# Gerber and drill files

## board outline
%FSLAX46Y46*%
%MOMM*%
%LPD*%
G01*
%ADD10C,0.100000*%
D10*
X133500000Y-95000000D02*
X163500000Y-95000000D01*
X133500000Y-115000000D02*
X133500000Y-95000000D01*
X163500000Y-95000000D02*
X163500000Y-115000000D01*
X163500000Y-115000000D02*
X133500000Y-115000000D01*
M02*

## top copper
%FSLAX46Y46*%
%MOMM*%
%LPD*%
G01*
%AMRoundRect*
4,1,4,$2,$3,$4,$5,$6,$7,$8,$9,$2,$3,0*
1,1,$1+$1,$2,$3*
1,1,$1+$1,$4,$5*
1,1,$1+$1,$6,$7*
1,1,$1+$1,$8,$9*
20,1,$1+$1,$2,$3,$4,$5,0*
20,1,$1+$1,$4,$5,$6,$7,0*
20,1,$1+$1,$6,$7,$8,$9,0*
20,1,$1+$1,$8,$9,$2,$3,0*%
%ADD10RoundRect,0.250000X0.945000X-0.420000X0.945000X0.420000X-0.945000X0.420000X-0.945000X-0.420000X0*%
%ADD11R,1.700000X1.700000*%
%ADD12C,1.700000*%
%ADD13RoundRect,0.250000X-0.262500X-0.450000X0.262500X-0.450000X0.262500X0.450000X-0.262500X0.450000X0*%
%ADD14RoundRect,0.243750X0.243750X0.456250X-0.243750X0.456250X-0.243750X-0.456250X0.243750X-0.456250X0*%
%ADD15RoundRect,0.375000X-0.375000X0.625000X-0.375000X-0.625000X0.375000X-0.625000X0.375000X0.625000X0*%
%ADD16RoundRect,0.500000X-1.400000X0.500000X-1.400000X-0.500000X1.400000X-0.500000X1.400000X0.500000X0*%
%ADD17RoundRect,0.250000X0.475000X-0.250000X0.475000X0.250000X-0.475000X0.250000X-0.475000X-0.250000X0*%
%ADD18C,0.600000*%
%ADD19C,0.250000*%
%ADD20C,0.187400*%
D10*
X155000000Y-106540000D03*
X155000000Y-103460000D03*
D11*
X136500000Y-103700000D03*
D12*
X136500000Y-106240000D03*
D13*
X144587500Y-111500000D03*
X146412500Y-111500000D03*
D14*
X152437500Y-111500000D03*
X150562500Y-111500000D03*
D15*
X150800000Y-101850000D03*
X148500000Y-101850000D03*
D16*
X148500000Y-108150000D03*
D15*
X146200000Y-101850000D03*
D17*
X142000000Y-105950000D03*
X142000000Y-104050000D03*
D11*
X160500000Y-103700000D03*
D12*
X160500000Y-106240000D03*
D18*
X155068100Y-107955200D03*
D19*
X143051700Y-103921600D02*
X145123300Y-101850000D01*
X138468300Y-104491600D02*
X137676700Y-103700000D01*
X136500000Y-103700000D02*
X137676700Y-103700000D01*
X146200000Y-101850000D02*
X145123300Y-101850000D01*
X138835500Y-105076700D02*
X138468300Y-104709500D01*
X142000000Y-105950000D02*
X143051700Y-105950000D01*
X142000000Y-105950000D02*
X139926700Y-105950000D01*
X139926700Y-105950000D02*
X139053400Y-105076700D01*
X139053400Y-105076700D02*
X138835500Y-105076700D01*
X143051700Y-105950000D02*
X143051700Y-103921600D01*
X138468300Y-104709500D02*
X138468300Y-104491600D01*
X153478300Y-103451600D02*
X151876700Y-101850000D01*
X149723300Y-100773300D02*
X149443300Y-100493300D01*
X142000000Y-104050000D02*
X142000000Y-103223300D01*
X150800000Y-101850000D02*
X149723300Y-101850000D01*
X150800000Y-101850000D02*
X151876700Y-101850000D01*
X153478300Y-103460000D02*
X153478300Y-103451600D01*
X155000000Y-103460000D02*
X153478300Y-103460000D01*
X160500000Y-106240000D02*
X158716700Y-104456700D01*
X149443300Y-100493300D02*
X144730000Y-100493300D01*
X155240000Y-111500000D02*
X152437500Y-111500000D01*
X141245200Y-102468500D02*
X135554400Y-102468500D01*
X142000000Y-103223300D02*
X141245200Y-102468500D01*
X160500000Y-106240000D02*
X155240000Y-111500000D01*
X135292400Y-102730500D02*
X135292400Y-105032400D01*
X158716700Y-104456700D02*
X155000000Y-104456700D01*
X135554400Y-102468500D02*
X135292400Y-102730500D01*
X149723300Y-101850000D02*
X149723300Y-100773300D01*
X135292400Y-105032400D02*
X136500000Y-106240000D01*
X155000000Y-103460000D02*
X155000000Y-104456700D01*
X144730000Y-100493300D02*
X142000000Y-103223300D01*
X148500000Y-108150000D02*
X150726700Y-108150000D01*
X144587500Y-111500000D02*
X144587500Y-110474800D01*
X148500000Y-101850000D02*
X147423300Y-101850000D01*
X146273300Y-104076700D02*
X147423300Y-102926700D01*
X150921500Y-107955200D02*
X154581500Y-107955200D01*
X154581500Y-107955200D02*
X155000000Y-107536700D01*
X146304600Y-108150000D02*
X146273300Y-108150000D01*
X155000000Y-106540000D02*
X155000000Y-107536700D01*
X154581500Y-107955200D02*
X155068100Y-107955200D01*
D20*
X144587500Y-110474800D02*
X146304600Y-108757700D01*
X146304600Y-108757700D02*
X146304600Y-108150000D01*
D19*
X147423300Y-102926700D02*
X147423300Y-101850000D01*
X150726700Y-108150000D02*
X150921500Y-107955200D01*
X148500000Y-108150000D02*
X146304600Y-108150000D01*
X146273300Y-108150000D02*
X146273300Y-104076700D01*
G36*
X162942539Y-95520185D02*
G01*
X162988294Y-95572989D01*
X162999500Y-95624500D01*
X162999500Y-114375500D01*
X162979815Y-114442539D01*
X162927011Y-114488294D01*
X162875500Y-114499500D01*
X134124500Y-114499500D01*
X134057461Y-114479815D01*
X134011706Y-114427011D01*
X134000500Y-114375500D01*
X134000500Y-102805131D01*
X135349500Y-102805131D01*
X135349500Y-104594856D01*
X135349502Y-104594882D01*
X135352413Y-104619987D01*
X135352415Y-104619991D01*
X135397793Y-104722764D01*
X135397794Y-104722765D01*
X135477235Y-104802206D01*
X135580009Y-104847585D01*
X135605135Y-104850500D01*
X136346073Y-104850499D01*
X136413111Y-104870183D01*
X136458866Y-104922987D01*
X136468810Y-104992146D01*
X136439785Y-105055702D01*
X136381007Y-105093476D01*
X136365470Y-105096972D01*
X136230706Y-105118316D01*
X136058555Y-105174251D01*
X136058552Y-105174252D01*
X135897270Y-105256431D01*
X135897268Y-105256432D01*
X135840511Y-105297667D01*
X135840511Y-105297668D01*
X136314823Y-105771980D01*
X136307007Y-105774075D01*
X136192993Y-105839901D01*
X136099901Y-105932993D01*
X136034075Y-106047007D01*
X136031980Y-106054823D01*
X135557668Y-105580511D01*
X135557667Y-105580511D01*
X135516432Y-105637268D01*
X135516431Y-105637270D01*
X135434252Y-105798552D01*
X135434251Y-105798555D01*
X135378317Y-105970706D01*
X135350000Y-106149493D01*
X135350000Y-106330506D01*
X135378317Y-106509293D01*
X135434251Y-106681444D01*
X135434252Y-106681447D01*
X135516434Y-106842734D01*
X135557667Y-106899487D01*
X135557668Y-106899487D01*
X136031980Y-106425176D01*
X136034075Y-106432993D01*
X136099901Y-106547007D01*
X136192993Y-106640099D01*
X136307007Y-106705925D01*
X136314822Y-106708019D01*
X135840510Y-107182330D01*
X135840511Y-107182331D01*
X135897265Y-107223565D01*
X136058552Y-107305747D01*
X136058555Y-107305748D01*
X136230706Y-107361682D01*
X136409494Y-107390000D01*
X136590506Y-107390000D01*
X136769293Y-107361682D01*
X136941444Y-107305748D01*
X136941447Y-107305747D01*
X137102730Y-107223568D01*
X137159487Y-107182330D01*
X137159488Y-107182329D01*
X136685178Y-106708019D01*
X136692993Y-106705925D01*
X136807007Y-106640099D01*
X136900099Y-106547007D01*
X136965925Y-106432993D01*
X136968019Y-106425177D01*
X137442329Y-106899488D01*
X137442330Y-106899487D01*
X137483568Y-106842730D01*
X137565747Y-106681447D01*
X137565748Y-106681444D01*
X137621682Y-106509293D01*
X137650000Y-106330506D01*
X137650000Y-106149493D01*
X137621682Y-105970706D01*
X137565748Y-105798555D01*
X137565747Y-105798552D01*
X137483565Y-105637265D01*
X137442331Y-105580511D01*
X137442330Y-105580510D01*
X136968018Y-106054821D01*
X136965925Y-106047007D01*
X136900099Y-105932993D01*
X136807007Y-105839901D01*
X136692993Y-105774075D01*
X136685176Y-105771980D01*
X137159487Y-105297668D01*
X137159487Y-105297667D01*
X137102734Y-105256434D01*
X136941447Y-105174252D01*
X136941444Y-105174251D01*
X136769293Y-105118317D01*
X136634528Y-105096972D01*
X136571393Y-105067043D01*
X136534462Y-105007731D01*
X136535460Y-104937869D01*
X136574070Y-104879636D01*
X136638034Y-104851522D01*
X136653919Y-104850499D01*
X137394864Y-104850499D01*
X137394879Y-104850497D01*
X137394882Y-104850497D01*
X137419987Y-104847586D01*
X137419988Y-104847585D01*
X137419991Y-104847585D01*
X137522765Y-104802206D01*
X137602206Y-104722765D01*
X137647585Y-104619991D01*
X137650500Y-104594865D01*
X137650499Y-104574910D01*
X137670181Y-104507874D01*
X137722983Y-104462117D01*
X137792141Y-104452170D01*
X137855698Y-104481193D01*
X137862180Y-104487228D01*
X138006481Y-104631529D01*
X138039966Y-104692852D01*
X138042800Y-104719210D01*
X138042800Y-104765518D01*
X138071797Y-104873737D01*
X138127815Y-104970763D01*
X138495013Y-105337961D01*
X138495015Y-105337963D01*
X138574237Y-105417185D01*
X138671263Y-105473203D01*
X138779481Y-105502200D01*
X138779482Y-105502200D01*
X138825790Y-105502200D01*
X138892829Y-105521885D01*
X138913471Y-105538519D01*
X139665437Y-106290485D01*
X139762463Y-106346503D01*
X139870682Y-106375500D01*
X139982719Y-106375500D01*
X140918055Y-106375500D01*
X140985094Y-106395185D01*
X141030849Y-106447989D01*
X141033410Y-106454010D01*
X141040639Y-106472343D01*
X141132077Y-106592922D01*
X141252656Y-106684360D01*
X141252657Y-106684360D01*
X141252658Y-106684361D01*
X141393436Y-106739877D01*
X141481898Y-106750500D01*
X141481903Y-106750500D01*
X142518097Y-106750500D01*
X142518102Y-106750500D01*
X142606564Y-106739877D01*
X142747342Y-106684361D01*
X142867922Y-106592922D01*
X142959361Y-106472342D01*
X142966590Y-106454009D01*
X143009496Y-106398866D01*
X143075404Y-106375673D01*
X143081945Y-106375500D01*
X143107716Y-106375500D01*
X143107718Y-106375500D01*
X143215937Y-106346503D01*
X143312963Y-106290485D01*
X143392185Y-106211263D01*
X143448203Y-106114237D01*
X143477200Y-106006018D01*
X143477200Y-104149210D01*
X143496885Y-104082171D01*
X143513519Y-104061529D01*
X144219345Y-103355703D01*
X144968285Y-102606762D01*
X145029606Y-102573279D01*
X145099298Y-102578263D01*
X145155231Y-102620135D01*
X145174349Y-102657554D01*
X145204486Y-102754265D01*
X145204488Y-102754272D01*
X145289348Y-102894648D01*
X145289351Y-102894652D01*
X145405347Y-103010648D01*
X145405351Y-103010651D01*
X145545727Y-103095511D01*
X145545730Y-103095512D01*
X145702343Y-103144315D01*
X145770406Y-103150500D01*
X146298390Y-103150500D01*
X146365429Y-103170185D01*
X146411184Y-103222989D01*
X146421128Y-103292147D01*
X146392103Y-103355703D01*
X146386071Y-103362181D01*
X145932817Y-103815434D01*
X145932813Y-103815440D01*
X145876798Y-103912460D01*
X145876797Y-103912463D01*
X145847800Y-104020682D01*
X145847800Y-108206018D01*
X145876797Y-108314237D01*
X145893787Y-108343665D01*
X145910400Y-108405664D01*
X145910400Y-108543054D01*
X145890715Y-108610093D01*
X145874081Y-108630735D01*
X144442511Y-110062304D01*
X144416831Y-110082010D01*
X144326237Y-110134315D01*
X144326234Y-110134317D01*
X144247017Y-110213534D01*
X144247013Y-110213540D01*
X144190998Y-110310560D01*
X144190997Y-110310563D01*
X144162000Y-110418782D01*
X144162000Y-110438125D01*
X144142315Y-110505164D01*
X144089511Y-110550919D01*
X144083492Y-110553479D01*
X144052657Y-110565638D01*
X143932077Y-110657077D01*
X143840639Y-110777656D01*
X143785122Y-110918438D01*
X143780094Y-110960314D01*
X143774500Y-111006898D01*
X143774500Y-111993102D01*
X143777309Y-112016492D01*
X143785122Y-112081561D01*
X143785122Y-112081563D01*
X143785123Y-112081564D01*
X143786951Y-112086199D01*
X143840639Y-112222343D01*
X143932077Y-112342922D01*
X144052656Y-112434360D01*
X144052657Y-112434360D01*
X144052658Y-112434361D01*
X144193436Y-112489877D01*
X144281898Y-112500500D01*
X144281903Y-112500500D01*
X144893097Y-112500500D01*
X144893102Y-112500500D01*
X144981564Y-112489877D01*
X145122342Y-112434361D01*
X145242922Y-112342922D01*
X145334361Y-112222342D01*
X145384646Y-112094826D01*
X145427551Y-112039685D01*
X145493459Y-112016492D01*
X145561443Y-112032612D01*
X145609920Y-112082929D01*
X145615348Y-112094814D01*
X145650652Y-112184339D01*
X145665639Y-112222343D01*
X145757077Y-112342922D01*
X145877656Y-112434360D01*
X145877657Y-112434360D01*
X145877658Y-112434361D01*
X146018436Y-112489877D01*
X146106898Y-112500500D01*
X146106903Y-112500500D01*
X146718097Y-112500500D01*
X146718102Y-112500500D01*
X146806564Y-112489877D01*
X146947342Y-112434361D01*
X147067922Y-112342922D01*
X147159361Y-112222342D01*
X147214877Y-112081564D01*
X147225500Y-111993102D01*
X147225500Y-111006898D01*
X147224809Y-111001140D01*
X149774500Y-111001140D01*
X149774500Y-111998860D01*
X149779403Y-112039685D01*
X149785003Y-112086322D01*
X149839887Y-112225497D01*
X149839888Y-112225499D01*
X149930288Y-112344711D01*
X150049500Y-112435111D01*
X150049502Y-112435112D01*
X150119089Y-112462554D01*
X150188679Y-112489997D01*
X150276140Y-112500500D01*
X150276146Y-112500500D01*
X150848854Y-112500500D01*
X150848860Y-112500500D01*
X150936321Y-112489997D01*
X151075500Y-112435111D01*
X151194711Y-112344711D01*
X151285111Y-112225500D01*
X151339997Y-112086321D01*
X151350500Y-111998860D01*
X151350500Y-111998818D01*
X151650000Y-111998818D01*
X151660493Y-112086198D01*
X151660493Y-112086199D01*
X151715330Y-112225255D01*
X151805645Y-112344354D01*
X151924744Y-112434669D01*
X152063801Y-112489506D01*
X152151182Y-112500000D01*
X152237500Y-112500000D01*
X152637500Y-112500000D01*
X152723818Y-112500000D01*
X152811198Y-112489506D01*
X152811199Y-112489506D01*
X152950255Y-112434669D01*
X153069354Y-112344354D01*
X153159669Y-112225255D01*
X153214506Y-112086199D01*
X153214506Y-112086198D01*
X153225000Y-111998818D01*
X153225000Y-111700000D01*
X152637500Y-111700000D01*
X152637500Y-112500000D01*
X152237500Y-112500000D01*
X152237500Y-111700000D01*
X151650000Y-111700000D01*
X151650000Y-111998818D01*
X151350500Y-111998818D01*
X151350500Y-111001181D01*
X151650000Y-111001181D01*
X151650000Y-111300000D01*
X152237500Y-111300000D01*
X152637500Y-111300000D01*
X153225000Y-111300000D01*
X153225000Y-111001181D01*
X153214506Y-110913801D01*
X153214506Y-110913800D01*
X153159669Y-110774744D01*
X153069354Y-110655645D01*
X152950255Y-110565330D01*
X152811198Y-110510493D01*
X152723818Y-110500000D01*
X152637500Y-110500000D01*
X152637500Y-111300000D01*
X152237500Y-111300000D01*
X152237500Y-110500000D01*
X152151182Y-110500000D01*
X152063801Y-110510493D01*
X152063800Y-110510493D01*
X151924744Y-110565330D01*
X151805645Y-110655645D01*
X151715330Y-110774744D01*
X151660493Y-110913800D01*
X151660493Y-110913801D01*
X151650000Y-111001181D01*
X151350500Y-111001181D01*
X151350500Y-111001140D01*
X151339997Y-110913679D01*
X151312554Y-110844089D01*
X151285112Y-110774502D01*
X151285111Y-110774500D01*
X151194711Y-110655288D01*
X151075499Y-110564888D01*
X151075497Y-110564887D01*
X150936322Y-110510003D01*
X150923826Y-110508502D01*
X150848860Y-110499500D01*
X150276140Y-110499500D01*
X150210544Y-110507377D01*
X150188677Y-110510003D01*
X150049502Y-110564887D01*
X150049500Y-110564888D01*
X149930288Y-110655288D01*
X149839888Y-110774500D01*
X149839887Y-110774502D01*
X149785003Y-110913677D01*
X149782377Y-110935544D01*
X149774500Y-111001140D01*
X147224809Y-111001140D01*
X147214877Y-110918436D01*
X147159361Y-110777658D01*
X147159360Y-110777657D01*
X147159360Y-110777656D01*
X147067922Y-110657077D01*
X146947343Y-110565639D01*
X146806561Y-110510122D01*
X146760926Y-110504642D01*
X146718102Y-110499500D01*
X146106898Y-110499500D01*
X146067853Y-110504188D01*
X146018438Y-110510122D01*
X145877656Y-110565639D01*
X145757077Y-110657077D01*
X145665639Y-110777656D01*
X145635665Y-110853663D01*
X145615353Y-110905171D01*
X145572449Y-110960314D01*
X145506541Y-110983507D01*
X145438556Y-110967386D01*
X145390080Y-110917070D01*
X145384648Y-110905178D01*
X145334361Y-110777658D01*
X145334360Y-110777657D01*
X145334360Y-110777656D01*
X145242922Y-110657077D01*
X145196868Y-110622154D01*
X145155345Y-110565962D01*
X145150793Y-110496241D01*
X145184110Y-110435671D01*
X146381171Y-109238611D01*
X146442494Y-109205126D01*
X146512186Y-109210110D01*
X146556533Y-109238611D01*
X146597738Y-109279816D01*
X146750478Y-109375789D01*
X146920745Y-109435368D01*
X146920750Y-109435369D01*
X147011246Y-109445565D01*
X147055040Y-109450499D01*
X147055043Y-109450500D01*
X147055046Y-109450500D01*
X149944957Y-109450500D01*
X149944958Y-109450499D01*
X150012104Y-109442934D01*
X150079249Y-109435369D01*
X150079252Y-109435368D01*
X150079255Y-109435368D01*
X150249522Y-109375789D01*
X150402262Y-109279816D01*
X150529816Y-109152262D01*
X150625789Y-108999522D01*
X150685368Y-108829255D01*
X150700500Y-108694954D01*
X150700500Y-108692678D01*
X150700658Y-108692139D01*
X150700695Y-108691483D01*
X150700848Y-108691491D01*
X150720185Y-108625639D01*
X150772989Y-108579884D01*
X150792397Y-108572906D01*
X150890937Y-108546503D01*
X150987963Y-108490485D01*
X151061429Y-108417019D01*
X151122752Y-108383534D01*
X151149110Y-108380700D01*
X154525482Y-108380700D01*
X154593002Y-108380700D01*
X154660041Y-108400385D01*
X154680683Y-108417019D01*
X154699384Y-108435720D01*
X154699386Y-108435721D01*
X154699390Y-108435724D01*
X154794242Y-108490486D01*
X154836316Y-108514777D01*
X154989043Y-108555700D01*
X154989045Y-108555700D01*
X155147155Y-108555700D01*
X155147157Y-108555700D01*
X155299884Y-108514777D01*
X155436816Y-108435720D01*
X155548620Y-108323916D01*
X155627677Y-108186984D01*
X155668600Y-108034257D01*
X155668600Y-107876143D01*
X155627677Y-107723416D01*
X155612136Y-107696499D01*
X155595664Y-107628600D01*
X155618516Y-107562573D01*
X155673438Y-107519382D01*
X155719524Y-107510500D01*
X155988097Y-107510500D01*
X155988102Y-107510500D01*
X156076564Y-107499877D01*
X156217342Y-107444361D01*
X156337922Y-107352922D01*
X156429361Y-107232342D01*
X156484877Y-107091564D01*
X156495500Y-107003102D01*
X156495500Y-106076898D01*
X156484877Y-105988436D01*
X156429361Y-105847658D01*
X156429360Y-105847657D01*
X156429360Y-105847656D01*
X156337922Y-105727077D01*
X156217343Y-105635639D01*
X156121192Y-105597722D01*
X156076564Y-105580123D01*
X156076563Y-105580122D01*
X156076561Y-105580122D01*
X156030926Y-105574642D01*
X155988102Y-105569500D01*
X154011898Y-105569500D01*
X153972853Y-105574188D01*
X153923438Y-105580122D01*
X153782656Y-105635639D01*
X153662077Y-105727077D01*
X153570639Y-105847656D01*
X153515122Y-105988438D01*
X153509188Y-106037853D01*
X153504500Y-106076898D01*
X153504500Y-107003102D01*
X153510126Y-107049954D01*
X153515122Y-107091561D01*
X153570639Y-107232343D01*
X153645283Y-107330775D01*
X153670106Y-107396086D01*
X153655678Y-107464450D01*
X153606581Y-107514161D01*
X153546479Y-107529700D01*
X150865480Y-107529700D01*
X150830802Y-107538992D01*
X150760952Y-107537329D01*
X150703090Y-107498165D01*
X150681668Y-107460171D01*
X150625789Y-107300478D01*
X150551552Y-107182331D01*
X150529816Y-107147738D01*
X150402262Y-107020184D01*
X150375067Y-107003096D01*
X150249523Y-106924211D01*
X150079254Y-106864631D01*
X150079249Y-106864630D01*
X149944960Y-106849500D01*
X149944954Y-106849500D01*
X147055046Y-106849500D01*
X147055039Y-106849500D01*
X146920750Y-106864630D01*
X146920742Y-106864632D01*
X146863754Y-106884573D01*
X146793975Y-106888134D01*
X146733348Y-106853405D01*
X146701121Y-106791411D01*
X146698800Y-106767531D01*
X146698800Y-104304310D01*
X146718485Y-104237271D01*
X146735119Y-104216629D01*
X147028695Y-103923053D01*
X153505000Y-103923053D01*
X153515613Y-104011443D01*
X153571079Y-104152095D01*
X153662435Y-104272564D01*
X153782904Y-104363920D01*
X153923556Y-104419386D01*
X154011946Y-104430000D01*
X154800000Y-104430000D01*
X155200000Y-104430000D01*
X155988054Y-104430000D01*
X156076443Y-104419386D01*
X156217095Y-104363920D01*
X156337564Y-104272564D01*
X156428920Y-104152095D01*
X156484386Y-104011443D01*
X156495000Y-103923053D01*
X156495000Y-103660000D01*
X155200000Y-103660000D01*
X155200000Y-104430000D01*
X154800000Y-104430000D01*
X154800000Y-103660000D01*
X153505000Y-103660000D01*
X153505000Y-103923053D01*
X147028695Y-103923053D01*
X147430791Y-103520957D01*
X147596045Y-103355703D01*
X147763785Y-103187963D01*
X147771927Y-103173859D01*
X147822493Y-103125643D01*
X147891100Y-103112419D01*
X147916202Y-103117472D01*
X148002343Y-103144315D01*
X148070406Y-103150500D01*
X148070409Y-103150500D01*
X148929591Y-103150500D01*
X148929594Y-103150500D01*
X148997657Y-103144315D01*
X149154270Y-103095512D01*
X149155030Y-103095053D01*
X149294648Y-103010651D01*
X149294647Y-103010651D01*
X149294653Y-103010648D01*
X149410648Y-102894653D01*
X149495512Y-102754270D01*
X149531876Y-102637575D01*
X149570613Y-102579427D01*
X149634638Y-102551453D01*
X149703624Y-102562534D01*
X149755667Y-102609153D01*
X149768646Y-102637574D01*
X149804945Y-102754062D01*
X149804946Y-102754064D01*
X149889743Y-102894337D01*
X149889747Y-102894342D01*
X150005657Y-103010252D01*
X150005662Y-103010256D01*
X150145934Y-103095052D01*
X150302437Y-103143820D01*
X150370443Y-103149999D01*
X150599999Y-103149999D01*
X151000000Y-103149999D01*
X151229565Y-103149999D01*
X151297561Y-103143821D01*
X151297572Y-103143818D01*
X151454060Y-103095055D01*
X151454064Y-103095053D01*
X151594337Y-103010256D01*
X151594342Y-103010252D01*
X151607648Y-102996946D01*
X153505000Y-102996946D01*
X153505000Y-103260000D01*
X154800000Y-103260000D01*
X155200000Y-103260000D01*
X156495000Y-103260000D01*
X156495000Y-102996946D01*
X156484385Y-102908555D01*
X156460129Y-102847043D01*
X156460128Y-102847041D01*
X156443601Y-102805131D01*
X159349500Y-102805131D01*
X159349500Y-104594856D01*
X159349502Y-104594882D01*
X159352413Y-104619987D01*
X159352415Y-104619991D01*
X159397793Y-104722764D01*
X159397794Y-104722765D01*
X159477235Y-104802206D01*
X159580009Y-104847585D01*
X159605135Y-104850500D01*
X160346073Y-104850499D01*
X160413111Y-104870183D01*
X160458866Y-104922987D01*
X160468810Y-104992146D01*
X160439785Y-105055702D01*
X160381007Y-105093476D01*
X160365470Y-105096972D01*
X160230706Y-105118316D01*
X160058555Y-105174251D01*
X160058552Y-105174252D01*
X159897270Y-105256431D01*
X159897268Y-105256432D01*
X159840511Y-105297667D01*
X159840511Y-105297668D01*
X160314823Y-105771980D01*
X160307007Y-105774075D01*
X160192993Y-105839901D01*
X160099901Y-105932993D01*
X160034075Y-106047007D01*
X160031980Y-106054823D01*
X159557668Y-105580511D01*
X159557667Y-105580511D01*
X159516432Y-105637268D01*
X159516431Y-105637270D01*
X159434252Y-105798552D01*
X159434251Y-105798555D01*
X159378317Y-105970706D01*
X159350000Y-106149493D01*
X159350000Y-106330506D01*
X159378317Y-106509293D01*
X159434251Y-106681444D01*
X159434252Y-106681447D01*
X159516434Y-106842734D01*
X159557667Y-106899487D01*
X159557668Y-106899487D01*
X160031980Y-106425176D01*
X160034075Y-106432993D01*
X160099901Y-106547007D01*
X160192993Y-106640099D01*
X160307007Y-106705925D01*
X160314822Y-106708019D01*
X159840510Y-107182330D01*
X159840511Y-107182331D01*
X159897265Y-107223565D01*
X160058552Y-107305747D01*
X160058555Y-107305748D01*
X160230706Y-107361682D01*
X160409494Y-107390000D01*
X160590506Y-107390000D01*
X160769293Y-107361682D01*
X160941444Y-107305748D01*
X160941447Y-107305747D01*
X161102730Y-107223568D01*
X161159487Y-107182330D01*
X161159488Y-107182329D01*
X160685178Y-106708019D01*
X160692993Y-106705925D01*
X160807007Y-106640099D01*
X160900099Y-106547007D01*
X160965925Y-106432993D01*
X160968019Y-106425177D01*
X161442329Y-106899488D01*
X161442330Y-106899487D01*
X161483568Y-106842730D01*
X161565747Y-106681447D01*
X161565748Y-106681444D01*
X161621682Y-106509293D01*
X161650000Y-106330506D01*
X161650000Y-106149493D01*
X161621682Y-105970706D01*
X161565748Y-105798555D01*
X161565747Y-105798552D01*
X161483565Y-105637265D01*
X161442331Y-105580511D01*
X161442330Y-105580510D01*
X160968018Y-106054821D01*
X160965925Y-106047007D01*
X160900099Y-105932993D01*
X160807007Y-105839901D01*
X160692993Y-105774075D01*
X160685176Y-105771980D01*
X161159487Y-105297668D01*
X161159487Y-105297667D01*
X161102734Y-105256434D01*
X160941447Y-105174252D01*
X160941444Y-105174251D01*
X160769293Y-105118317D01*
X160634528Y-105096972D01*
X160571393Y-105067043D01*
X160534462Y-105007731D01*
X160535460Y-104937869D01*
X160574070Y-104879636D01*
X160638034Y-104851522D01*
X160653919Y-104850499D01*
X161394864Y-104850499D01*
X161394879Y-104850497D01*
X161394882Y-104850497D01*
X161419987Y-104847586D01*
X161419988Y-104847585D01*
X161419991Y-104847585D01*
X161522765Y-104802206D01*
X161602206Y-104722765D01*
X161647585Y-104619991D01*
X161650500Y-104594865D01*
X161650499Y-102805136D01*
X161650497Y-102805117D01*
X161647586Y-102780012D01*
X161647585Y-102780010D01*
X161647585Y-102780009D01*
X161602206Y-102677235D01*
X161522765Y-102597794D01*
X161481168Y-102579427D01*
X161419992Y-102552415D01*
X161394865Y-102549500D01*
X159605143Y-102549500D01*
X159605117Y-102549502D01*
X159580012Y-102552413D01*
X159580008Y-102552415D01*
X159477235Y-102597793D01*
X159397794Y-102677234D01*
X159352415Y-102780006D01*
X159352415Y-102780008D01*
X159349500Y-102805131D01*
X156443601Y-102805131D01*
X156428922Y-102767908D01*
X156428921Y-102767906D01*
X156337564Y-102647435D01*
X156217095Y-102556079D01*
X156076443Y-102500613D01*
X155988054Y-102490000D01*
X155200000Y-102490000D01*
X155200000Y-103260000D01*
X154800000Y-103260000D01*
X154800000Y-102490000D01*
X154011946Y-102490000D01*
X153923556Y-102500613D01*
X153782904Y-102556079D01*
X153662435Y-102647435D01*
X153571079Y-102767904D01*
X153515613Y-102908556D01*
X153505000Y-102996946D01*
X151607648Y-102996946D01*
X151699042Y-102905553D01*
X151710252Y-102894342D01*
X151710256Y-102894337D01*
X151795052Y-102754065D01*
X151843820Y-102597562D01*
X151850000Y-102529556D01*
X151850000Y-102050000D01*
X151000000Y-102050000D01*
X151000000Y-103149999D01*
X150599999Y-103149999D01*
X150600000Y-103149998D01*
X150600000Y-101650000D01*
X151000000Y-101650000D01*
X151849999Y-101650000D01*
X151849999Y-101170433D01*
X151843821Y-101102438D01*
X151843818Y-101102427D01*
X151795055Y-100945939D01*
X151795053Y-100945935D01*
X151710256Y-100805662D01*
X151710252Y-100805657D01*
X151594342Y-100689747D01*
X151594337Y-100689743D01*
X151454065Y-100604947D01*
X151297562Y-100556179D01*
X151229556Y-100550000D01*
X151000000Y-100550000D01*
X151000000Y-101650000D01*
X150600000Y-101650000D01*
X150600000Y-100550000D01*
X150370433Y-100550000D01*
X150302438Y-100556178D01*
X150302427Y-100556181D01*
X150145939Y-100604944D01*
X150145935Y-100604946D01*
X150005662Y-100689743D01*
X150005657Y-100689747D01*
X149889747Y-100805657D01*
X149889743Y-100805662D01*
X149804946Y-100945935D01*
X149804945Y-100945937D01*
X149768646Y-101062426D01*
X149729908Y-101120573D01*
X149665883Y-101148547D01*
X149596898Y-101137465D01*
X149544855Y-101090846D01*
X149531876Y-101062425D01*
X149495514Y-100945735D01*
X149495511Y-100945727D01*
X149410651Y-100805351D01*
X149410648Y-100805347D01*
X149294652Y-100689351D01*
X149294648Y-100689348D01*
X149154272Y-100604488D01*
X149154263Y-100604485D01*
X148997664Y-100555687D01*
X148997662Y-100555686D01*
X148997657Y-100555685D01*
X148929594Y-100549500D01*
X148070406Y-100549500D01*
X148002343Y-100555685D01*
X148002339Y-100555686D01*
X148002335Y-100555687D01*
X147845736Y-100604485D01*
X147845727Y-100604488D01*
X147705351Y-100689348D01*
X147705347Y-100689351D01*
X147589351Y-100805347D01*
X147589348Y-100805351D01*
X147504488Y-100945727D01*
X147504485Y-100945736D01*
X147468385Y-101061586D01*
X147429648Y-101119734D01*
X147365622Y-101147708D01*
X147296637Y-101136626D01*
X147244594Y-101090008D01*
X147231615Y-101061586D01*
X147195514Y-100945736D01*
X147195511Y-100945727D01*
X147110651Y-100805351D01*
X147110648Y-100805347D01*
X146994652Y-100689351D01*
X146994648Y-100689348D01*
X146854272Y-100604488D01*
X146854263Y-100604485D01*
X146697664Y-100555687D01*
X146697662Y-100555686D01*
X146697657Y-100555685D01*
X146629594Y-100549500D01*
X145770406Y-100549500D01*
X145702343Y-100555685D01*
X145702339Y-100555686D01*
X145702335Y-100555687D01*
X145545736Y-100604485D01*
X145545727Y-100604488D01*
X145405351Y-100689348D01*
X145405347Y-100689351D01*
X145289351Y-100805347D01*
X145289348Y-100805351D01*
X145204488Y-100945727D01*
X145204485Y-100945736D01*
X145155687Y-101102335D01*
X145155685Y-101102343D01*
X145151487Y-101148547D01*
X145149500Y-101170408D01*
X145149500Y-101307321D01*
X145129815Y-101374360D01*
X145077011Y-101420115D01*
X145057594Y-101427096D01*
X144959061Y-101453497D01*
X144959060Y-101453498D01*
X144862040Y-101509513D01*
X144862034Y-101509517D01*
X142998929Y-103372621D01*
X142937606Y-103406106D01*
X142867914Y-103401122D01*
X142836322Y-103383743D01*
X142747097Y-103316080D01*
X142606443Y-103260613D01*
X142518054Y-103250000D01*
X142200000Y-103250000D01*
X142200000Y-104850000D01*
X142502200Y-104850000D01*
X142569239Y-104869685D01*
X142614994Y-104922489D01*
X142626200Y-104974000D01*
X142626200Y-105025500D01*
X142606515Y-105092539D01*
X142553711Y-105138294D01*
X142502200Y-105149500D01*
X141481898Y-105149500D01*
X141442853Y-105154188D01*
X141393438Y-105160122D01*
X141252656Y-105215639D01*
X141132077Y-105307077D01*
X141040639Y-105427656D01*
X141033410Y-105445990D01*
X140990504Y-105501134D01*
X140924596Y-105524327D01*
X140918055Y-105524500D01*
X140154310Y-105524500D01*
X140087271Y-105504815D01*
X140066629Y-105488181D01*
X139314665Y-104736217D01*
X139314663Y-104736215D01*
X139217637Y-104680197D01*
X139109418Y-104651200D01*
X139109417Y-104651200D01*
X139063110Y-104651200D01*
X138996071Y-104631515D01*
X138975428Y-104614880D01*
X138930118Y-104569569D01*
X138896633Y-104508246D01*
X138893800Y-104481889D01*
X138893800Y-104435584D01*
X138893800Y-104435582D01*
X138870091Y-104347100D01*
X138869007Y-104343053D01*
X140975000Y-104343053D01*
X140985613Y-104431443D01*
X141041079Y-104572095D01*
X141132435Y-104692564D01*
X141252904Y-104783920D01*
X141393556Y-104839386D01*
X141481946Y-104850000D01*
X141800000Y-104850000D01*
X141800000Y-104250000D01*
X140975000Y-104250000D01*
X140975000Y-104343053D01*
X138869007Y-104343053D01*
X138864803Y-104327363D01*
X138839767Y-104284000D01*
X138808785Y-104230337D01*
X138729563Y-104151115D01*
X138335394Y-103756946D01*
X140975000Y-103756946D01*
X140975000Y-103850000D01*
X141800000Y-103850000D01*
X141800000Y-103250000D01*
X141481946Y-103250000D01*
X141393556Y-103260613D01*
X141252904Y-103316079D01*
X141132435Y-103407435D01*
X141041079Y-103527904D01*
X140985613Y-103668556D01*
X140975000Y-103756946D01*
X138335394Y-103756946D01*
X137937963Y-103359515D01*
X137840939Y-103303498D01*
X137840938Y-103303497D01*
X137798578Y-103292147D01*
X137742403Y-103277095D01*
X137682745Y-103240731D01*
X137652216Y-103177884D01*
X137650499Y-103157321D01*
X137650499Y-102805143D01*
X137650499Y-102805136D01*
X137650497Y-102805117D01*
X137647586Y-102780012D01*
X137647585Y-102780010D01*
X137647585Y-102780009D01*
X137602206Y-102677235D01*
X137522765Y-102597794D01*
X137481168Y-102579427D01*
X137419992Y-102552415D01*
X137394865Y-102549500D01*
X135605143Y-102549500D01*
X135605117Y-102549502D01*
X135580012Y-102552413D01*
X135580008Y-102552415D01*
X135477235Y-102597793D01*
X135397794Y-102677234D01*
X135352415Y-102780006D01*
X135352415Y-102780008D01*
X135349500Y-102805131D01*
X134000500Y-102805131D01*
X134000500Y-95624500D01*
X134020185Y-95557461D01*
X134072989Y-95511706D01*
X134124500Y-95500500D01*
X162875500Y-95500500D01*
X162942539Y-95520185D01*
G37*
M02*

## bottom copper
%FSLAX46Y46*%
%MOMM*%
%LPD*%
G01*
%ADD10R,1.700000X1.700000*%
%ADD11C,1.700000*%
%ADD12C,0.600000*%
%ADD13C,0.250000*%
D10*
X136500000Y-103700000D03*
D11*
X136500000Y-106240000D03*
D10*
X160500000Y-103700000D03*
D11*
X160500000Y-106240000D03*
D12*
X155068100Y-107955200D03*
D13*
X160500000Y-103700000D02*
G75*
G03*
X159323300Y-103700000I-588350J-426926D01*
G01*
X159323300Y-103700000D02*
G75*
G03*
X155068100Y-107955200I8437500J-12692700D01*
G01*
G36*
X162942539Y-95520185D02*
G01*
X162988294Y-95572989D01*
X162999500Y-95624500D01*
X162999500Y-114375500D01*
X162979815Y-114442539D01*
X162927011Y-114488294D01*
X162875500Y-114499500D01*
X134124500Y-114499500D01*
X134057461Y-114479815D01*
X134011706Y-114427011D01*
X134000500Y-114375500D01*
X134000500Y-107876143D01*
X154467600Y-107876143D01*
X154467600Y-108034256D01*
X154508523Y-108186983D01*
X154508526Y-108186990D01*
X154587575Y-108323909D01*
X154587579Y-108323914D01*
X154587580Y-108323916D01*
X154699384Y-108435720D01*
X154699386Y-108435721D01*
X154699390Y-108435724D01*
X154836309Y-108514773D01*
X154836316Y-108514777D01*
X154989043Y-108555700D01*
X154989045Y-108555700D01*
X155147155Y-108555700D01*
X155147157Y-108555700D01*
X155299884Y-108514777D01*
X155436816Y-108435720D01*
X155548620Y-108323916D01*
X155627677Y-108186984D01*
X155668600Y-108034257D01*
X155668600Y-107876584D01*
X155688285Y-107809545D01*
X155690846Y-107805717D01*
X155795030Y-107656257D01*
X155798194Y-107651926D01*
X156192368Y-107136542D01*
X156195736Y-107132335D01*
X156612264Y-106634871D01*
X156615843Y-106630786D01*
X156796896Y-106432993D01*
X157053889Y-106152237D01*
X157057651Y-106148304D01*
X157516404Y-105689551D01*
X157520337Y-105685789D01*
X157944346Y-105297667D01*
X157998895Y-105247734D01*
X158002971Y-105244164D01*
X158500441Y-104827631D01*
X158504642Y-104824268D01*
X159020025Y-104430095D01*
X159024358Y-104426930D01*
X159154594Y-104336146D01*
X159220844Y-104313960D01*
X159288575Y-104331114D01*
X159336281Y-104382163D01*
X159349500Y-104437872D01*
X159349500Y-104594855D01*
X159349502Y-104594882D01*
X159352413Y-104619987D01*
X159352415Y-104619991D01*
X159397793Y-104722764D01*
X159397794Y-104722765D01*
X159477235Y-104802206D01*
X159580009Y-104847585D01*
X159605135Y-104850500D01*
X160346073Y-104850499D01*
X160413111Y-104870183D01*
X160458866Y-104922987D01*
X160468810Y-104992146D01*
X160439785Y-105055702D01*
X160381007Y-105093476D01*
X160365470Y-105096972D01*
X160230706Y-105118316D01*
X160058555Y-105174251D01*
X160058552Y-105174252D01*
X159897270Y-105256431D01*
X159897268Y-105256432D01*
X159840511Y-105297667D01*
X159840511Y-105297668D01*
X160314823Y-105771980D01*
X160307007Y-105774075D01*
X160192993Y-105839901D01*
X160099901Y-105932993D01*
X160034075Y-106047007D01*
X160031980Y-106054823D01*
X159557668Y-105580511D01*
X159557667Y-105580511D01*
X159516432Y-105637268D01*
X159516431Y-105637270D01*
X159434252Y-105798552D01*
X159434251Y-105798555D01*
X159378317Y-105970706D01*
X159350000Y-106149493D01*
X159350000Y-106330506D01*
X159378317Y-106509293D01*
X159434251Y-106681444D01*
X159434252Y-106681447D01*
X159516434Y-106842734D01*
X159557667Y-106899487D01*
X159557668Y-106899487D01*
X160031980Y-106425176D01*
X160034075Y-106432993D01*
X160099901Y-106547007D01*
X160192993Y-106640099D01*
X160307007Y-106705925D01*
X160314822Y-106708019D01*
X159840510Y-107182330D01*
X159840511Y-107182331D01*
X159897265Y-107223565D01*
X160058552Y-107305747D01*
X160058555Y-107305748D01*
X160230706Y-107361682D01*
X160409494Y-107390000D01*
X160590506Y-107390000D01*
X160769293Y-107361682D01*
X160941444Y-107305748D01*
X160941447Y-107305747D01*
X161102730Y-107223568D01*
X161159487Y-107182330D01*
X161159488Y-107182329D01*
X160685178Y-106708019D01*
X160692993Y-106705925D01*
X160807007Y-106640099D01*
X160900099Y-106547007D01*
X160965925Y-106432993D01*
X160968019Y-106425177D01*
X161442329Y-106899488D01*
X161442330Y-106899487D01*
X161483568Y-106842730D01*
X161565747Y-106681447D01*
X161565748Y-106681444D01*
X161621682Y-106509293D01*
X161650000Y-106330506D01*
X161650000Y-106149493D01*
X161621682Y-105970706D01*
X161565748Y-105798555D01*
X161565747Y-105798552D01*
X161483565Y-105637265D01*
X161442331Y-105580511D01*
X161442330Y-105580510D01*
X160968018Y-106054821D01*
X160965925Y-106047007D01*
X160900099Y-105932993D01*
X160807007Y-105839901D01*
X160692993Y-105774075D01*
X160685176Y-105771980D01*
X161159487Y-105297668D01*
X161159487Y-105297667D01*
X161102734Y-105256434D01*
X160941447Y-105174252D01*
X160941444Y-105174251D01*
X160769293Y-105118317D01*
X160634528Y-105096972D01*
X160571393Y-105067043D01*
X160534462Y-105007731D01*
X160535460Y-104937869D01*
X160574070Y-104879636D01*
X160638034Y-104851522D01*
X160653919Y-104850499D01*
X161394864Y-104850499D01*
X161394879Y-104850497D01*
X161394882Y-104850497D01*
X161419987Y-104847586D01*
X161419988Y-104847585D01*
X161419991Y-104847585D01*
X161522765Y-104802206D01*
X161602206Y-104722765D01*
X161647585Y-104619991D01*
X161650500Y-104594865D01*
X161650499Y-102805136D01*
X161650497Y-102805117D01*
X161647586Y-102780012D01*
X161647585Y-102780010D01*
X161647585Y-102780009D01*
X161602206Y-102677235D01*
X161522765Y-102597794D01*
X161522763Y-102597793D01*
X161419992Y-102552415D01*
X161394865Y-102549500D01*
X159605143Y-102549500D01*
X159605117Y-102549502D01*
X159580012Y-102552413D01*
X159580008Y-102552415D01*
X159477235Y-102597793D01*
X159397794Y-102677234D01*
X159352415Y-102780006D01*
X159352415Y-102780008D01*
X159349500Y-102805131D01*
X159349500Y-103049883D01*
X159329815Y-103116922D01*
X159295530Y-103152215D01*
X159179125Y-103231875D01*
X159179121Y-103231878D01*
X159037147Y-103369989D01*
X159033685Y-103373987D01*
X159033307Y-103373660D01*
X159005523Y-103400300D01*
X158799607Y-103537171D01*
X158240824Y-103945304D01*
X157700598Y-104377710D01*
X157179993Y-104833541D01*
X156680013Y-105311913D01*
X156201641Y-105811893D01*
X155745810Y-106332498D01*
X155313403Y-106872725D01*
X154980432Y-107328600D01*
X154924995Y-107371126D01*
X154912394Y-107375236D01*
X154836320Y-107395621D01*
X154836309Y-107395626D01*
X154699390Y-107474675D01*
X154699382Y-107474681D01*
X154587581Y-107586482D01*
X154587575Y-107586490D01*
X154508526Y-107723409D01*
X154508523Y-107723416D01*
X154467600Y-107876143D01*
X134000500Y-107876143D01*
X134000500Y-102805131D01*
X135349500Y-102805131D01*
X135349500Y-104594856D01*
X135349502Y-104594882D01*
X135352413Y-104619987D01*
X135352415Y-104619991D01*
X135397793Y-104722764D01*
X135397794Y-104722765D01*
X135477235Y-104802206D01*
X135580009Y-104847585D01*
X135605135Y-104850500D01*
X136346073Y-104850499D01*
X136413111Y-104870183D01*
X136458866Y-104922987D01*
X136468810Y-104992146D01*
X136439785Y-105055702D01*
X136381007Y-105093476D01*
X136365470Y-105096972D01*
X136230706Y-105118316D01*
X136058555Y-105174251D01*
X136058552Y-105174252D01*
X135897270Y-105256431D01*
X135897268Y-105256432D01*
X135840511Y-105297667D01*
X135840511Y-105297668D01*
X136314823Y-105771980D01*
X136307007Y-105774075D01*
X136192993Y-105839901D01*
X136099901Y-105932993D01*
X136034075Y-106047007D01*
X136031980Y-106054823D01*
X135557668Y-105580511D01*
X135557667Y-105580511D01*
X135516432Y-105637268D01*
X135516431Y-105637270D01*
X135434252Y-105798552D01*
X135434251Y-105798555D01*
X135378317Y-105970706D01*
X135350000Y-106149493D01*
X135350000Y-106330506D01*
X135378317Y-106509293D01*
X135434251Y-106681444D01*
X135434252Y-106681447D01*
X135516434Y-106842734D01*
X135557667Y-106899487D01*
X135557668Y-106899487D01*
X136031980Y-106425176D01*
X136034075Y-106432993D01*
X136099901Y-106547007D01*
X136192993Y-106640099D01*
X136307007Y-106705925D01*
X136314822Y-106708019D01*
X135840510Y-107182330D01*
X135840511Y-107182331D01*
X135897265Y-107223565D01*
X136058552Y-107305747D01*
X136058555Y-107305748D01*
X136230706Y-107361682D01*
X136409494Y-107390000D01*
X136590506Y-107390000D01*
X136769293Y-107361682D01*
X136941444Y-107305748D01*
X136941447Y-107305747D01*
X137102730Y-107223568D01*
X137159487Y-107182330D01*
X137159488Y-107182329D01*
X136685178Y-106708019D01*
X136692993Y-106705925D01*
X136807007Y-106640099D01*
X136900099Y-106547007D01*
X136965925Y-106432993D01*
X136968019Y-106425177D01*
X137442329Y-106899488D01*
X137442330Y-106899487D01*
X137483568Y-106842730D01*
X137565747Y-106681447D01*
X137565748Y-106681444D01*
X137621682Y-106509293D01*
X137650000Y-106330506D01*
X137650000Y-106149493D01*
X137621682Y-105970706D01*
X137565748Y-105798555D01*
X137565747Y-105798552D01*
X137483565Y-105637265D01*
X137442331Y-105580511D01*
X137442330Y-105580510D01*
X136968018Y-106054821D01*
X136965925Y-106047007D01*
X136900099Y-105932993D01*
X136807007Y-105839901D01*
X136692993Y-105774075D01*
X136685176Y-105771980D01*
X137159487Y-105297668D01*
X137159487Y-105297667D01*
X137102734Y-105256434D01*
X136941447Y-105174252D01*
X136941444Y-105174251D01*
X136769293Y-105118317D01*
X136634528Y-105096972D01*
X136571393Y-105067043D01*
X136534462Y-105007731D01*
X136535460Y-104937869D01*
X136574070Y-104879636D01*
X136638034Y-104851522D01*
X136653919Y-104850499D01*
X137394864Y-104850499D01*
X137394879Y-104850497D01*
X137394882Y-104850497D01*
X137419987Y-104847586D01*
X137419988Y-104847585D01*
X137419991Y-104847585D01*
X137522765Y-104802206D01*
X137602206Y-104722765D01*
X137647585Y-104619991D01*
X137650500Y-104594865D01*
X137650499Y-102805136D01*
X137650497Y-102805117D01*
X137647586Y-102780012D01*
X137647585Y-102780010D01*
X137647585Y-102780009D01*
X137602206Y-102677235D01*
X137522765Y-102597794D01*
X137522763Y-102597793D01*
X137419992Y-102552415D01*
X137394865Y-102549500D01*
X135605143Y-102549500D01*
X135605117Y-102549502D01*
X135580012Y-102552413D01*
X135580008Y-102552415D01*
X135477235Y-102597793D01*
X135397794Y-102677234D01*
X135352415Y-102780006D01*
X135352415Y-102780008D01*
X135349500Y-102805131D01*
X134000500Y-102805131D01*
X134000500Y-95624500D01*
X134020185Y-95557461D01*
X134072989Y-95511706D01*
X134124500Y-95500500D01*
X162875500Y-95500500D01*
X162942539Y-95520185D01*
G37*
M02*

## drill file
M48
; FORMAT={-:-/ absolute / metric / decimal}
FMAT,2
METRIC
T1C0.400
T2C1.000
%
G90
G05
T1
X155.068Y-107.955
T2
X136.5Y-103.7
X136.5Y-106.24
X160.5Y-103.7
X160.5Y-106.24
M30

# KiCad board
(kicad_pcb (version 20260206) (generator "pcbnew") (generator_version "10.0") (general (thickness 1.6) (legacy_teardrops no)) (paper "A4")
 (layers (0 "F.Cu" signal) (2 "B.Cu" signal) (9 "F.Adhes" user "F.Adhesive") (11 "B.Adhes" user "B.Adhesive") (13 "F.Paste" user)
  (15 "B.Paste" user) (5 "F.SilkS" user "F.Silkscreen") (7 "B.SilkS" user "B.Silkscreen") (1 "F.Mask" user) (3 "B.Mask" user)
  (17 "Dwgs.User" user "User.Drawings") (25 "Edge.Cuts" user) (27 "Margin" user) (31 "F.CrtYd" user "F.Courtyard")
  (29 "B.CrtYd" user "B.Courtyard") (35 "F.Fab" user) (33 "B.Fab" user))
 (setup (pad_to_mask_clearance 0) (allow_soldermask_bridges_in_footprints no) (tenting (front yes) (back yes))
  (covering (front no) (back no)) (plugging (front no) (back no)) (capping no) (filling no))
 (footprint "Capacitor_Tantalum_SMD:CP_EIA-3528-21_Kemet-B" (layer "F.Cu") (at 155 105 90)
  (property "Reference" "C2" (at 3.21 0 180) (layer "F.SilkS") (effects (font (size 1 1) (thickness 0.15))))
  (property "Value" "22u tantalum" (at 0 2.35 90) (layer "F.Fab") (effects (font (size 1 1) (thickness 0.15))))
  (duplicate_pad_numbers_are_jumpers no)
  (pad "1" smd roundrect (at -1.54 0 90) (size 1.34 2.39) (layers "F.Cu" "F.Mask" "F.Paste") (roundrect_rratio 0.186567) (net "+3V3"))
  (pad "2" smd roundrect (at 1.54 0 90) (size 1.34 2.39) (layers "F.Cu" "F.Mask" "F.Paste") (roundrect_rratio 0.186567) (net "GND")))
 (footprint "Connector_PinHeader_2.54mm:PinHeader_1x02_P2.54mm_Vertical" (layer "F.Cu") (at 136.5 103.7)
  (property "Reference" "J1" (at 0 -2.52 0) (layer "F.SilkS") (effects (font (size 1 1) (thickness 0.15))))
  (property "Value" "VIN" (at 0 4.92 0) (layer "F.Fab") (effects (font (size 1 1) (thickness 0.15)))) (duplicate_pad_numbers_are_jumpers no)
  (pad "1" thru_hole rect (at 0 0) (size 1.7 1.7) (drill 1) (layers "*.Cu" "*.Mask") (remove_unused_layers no) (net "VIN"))
  (pad "2" thru_hole circle (at 0 2.54) (size 1.7 1.7) (drill 1) (layers "*.Cu" "*.Mask") (remove_unused_layers no) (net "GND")))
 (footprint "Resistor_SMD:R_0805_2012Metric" (layer "F.Cu") (at 145.5 111.5)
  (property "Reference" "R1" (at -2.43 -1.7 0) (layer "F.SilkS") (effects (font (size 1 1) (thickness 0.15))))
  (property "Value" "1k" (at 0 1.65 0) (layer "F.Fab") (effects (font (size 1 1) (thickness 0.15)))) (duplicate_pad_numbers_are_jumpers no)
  (pad "1" smd roundrect (at -0.9125 0) (size 1.025 1.4) (layers "F.Cu" "F.Mask" "F.Paste") (roundrect_rratio 0.243902) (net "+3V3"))
  (pad "2" smd roundrect (at 0.9125 0) (size 1.025 1.4) (layers "F.Cu" "F.Mask" "F.Paste") (roundrect_rratio 0.243902) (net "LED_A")))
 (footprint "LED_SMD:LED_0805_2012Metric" (layer "F.Cu") (at 151.5 111.5 180)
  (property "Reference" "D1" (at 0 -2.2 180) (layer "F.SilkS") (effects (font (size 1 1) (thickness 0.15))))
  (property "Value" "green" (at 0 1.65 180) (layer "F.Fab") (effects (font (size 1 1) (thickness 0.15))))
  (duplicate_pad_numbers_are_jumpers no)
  (pad "1" smd roundrect (at -0.9375 0 180) (size 0.975 1.4) (layers "F.Cu" "F.Mask" "F.Paste") (roundrect_rratio 0.25) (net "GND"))
  (pad "2" smd roundrect (at 0.9375 0 180) (size 0.975 1.4) (layers "F.Cu" "F.Mask" "F.Paste") (roundrect_rratio 0.25) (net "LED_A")))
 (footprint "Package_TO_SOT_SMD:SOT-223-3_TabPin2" (layer "F.Cu") (at 148.5 105 -90)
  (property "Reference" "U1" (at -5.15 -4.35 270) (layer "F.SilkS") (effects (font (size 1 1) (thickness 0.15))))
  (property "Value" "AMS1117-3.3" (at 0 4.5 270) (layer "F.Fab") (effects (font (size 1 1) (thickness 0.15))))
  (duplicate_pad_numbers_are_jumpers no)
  (pad "1" smd roundrect (at -3.15 -2.3 270) (size 2 1.5) (layers "F.Cu" "F.Mask" "F.Paste") (roundrect_rratio 0.25) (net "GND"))
  (pad "2" smd roundrect (at -3.15 0 270) (size 2 1.5) (layers "F.Cu" "F.Mask" "F.Paste") (roundrect_rratio 0.25) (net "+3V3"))
  (pad "2" smd roundrect (at 3.15 0 270) (size 2 3.8) (layers "F.Cu" "F.Mask" "F.Paste") (roundrect_rratio 0.25) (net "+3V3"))
  (pad "3" smd roundrect (at -3.15 2.3 270) (size 2 1.5) (layers "F.Cu" "F.Mask" "F.Paste") (roundrect_rratio 0.25) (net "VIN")))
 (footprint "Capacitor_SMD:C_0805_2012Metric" (layer "F.Cu") (at 142 105 90)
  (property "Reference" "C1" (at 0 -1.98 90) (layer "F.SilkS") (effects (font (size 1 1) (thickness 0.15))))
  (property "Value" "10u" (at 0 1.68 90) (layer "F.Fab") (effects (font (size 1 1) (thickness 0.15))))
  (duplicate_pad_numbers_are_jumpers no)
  (pad "1" smd roundrect (at -0.95 0 90) (size 1 1.45) (layers "F.Cu" "F.Mask" "F.Paste") (roundrect_rratio 0.25) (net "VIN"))
  (pad "2" smd roundrect (at 0.95 0 90) (size 1 1.45) (layers "F.Cu" "F.Mask" "F.Paste") (roundrect_rratio 0.25) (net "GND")))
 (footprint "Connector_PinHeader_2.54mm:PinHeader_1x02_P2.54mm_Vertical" (layer "F.Cu") (at 160.5 103.7)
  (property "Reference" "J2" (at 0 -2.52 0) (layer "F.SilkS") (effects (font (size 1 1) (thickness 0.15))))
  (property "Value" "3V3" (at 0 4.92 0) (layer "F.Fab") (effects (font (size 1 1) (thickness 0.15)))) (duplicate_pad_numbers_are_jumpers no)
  (pad "1" thru_hole rect (at 0 0) (size 1.7 1.7) (drill 1) (layers "*.Cu" "*.Mask") (remove_unused_layers no) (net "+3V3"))
  (pad "2" thru_hole circle (at 0 2.54) (size 1.7 1.7) (drill 1) (layers "*.Cu" "*.Mask") (remove_unused_layers no) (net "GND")))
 (gr_line (start 133.5 95) (end 163.5 95) (stroke (width 0.1) (type default)) (layer "Edge.Cuts"))
 (gr_line (start 133.5 115) (end 133.5 95) (stroke (width 0.1) (type default)) (layer "Edge.Cuts"))
 (gr_line (start 163.5 95) (end 163.5 115) (stroke (width 0.1) (type default)) (layer "Edge.Cuts"))
 (gr_line (start 163.5 115) (end 133.5 115) (stroke (width 0.1) (type default)) (layer "Edge.Cuts"))
 (segment (start 143.0517 103.9216) (end 145.1233 101.85) (width 0.25) (layer "F.Cu") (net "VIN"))
 (segment (start 138.4683 104.4916) (end 137.6767 103.7) (width 0.25) (layer "F.Cu") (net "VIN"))
 (segment (start 136.5 103.7) (end 137.6767 103.7) (width 0.25) (layer "F.Cu") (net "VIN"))
 (segment (start 146.2 101.85) (end 145.1233 101.85) (width 0.25) (layer "F.Cu") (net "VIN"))
 (segment (start 138.8355 105.0767) (end 138.4683 104.7095) (width 0.25) (layer "F.Cu") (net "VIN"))
 (segment (start 142 105.95) (end 143.0517 105.95) (width 0.25) (layer "F.Cu") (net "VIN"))
 (segment (start 142 105.95) (end 139.9267 105.95) (width 0.25) (layer "F.Cu") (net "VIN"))
 (segment (start 139.9267 105.95) (end 139.0534 105.0767) (width 0.25) (layer "F.Cu") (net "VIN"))
 (segment (start 139.0534 105.0767) (end 138.8355 105.0767) (width 0.25) (layer "F.Cu") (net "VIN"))
 (segment (start 143.0517 105.95) (end 143.0517 103.9216) (width 0.25) (layer "F.Cu") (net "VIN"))
 (segment (start 138.4683 104.7095) (end 138.4683 104.4916) (width 0.25) (layer "F.Cu") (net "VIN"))
 (segment (start 153.4783 103.4516) (end 151.8767 101.85) (width 0.25) (layer "F.Cu") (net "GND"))
 (segment (start 149.7233 100.7733) (end 149.4433 100.4933) (width 0.25) (layer "F.Cu") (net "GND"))
 (segment (start 142 104.05) (end 142 103.2233) (width 0.25) (layer "F.Cu") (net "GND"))
 (segment (start 150.8 101.85) (end 149.7233 101.85) (width 0.25) (layer "F.Cu") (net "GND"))
 (segment (start 150.8 101.85) (end 151.8767 101.85) (width 0.25) (layer "F.Cu") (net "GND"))
 (segment (start 153.4783 103.46) (end 153.4783 103.4516) (width 0.25) (layer "F.Cu") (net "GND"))
 (segment (start 155 103.46) (end 153.4783 103.46) (width 0.25) (layer "F.Cu") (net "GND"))
 (segment (start 160.5 106.24) (end 158.7167 104.4567) (width 0.25) (layer "F.Cu") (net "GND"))
 (segment (start 149.4433 100.4933) (end 144.73 100.4933) (width 0.25) (layer "F.Cu") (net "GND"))
 (segment (start 155.24 111.5) (end 152.4375 111.5) (width 0.25) (layer "F.Cu") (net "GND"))
 (segment (start 141.2452 102.4685) (end 135.5544 102.4685) (width 0.25) (layer "F.Cu") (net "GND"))
 (segment (start 142 103.2233) (end 141.2452 102.4685) (width 0.25) (layer "F.Cu") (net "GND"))
 (segment (start 160.5 106.24) (end 155.24 111.5) (width 0.25) (layer "F.Cu") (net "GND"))
 (segment (start 135.2924 102.7305) (end 135.2924 105.0324) (width 0.25) (layer "F.Cu") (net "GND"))
 (segment (start 158.7167 104.4567) (end 155 104.4567) (width 0.25) (layer "F.Cu") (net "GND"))
 (segment (start 135.5544 102.4685) (end 135.2924 102.7305) (width 0.25) (layer "F.Cu") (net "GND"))
 (segment (start 149.7233 101.85) (end 149.7233 100.7733) (width 0.25) (layer "F.Cu") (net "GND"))
 (segment (start 135.2924 105.0324) (end 136.5 106.24) (width 0.25) (layer "F.Cu") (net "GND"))
 (segment (start 155 103.46) (end 155 104.4567) (width 0.25) (layer "F.Cu") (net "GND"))
 (segment (start 144.73 100.4933) (end 142 103.2233) (width 0.25) (layer "F.Cu") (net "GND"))
 (segment (start 148.5 108.15) (end 150.7267 108.15) (width 0.25) (layer "F.Cu") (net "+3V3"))
 (segment (start 144.5875 111.5) (end 144.5875 110.4748) (width 0.25) (layer "F.Cu") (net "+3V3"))
 (segment (start 148.5 101.85) (end 147.4233 101.85) (width 0.25) (layer "F.Cu") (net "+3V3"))
 (segment (start 146.2733 104.0767) (end 147.4233 102.9267) (width 0.25) (layer "F.Cu") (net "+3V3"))
 (segment (start 150.9215 107.9552) (end 154.5815 107.9552) (width 0.25) (layer "F.Cu") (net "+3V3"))
 (segment (start 154.5815 107.9552) (end 155 107.5367) (width 0.25) (layer "F.Cu") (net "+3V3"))
 (segment (start 146.3046 108.15) (end 146.2733 108.15) (width 0.25) (layer "F.Cu") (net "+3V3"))
 (segment (start 155 106.54) (end 155 107.5367) (width 0.25) (layer "F.Cu") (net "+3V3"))
 (segment (start 154.5815 107.9552) (end 155.0681 107.9552) (width 0.25) (layer "F.Cu") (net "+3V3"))
 (segment (start 144.5875 110.4748) (end 146.3046 108.7577) (width 0.1874) (layer "F.Cu") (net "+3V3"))
 (segment (start 146.3046 108.7577) (end 146.3046 108.15) (width 0.1874) (layer "F.Cu") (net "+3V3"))
 (segment (start 147.4233 102.9267) (end 147.4233 101.85) (width 0.25) (layer "F.Cu") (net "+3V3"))
 (segment (start 150.7267 108.15) (end 150.9215 107.9552) (width 0.25) (layer "F.Cu") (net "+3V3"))
 (segment (start 148.5 108.15) (end 146.3046 108.15) (width 0.25) (layer "F.Cu") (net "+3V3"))
 (segment (start 146.2733 108.15) (end 146.2733 104.0767) (width 0.25) (layer "F.Cu") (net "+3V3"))
 (via (at 155.0681 107.9552) (size 0.6) (drill 0.4) (layers "F.Cu" "B.Cu") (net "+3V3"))
 (arc (start 160.5 103.7) (mid 159.9117 103.4) (end 159.3233 103.7) (width 0.25) (layer "B.Cu") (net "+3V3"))
 (arc (start 159.3233 103.7) (mid 156.9836 105.6155) (end 155.0681 107.9552) (width 0.25) (layer "B.Cu") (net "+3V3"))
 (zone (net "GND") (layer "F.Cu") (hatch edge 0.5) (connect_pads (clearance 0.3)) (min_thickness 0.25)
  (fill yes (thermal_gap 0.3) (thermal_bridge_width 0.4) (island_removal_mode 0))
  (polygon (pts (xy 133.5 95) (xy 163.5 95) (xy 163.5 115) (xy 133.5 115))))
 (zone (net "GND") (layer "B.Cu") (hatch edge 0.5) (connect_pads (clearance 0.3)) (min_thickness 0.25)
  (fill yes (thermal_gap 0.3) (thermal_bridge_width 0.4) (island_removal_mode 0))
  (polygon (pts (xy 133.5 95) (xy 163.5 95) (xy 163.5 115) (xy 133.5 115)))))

